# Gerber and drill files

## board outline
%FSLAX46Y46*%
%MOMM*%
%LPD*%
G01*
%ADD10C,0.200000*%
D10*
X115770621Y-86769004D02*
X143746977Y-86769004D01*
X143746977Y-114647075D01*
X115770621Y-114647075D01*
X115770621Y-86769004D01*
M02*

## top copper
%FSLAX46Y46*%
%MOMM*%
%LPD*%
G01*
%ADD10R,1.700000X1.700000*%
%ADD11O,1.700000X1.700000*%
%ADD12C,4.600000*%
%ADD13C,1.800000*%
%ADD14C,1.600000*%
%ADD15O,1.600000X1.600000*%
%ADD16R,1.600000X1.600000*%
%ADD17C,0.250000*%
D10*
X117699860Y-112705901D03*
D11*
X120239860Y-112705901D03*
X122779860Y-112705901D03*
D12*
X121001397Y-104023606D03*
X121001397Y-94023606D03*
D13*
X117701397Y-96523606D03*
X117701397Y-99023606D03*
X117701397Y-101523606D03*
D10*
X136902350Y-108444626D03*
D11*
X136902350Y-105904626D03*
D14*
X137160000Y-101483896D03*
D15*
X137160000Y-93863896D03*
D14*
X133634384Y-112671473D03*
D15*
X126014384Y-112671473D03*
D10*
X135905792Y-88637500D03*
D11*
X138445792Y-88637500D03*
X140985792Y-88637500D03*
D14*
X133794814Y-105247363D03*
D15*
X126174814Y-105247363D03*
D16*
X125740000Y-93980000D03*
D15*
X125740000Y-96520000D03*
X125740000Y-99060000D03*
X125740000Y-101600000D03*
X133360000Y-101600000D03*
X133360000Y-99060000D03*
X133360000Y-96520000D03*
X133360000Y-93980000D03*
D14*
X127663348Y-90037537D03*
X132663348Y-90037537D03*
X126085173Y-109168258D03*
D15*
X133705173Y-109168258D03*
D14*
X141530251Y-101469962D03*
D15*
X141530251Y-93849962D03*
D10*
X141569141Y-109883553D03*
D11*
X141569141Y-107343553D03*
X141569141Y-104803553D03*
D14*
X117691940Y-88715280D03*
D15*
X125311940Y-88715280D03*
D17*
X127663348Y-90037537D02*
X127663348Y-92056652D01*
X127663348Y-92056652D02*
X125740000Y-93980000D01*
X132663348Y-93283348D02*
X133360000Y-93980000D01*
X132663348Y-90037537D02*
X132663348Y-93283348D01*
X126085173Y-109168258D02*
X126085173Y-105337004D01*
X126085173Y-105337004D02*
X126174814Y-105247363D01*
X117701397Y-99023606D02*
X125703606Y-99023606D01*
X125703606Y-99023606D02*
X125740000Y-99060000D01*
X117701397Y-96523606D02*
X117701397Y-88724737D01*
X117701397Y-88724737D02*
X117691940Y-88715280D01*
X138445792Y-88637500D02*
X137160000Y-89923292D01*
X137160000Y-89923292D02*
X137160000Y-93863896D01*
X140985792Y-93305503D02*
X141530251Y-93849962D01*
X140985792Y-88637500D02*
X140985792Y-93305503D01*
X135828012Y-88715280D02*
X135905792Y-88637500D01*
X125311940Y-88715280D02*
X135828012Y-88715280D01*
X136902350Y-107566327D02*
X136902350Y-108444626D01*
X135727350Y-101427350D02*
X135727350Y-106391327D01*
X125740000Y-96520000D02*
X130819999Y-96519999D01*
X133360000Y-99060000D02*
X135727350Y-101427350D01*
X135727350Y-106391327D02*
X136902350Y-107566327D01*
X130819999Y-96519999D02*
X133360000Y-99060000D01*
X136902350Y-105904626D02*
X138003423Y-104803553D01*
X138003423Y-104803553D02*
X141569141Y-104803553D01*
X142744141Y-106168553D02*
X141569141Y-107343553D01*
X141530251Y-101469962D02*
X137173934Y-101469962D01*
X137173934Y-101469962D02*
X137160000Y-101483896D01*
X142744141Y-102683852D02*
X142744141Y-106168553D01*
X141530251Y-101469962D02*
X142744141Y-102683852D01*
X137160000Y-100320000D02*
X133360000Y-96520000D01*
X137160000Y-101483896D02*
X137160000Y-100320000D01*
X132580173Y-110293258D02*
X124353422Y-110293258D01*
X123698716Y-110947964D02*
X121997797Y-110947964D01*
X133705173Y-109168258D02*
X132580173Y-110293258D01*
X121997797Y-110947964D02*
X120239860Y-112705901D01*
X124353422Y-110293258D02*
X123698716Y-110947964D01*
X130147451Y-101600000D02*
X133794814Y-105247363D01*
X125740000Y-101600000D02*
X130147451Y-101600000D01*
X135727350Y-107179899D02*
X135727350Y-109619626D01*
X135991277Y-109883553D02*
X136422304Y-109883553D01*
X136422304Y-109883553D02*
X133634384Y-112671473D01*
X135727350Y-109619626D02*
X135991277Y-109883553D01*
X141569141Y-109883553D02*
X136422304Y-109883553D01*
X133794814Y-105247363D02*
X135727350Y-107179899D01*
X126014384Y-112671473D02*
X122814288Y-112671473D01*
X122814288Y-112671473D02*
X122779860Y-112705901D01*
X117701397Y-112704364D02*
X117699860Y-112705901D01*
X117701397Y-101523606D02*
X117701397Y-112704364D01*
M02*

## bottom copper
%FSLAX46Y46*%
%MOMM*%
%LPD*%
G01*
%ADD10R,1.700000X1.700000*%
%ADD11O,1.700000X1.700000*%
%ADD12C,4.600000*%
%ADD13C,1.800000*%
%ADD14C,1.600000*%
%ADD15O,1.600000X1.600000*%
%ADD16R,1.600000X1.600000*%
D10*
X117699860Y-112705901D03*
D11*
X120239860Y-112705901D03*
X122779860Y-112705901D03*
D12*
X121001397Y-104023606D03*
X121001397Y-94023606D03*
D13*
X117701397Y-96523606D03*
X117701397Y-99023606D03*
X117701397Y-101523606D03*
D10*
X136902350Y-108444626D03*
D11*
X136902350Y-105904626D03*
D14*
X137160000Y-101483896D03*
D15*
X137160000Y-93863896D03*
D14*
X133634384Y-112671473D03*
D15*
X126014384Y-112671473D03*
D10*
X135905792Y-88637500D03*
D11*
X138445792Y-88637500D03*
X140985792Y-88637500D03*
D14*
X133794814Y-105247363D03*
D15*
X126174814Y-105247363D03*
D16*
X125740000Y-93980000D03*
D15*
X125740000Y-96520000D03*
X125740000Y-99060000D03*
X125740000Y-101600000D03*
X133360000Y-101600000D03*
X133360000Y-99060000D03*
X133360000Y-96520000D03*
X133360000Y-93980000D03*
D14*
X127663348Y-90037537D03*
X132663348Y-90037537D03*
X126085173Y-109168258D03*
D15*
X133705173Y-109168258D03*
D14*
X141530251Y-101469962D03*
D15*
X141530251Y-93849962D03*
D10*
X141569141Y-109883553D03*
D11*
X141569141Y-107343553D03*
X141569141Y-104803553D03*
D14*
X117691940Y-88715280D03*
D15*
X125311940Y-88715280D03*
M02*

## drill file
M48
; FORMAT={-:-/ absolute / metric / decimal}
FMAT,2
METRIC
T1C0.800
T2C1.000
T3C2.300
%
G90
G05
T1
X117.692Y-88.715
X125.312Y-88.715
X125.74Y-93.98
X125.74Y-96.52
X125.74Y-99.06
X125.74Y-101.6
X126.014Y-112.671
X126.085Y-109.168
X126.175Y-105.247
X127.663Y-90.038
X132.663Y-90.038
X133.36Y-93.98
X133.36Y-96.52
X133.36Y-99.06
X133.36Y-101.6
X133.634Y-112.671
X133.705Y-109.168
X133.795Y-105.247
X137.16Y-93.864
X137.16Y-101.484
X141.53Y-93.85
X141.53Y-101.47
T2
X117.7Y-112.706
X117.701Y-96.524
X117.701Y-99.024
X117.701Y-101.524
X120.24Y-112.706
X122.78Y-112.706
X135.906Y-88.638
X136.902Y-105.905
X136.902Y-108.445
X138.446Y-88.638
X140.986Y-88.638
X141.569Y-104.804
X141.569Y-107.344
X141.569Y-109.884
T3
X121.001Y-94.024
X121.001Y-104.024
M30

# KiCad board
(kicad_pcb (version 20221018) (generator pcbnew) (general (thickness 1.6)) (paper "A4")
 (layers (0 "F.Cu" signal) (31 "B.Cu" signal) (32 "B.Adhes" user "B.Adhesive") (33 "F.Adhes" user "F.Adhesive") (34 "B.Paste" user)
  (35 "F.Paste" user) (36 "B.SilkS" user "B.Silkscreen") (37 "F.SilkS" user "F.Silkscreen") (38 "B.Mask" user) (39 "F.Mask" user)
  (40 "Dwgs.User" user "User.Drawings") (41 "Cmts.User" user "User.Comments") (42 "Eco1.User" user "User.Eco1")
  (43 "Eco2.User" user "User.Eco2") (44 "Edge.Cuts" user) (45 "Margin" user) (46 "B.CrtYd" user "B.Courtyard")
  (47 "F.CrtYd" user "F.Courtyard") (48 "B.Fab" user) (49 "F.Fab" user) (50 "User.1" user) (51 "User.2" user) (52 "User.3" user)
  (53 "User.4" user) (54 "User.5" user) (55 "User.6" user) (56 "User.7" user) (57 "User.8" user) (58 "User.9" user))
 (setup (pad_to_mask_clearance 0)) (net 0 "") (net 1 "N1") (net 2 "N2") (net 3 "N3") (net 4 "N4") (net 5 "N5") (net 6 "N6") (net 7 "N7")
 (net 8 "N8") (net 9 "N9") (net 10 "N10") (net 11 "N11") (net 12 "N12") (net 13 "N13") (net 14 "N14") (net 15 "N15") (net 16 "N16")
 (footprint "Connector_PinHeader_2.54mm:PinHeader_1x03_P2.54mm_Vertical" (layer "F.Cu") (at 117.69986 112.705901 90)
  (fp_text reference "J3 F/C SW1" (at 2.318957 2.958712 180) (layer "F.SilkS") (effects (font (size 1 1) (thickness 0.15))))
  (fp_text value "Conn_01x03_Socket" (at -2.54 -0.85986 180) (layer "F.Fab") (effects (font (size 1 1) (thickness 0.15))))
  (pad "1" thru_hole rect (at 0 0 90) (size 1.7 1.7) (drill 1) (layers "*.Cu" "*.Mask") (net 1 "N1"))
  (pad "2" thru_hole oval (at 0 2.54 90) (size 1.7 1.7) (drill 1) (layers "*.Cu" "*.Mask") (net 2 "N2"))
  (pad "3" thru_hole oval (at 0 5.08 90) (size 1.7 1.7) (drill 1) (layers "*.Cu" "*.Mask") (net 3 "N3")))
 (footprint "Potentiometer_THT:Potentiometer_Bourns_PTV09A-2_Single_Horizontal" (layer "F.Cu") (at 117.701397 96.523606 180)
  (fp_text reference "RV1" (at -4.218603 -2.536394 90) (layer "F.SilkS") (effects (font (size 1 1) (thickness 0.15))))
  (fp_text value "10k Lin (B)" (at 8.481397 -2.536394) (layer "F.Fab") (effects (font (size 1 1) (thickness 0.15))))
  (pad "" thru_hole circle (at -3.3 -7.5 180) (size 4.6 4.6) (drill 2.3) (layers "*.Cu" "*.Mask"))
  (pad "" thru_hole circle (at -3.3 2.5 180) (size 4.6 4.6) (drill 2.3) (layers "*.Cu" "*.Mask"))
  (pad "1" thru_hole circle (at 0 0 180) (size 1.8 1.8) (drill 1) (layers "*.Cu" "*.Mask") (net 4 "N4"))
  (pad "2" thru_hole circle (at 0 -2.5 180) (size 1.8 1.8) (drill 1) (layers "*.Cu" "*.Mask") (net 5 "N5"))
  (pad "3" thru_hole circle (at 0 -5 180) (size 1.8 1.8) (drill 1) (layers "*.Cu" "*.Mask") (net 1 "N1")))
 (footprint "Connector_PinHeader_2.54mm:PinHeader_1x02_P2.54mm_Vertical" (layer "F.Cu") (at 136.90235 108.444626 180)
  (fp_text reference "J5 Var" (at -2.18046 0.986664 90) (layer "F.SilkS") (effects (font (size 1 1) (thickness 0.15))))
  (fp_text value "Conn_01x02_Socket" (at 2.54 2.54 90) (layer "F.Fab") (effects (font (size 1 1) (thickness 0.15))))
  (pad "1" thru_hole rect (at 0 0 180) (size 1.7 1.7) (drill 1) (layers "*.Cu" "*.Mask") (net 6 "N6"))
  (pad "2" thru_hole oval (at 0 2.54 180) (size 1.7 1.7) (drill 1) (layers "*.Cu" "*.Mask") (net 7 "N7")))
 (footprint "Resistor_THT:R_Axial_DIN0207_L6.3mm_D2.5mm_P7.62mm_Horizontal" (layer "F.Cu") (at 137.16 101.483896 90)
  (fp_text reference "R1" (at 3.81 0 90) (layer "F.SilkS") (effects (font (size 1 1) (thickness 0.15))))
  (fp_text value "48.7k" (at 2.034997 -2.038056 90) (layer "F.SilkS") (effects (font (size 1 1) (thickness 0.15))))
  (pad "1" thru_hole circle (at 0 0 90) (size 1.6 1.6) (drill 0.8) (layers "*.Cu" "*.Mask") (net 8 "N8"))
  (pad "2" thru_hole oval (at 7.62 0 90) (size 1.6 1.6) (drill 0.8) (layers "*.Cu" "*.Mask") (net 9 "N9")))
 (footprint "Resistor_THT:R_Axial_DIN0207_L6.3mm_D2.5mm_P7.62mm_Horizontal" (layer "F.Cu") (at 133.634384 112.671473 180)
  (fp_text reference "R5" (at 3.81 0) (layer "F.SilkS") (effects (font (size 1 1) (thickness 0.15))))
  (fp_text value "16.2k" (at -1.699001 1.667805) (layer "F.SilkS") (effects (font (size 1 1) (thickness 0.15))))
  (pad "1" thru_hole circle (at 0 0 180) (size 1.6 1.6) (drill 0.8) (layers "*.Cu" "*.Mask") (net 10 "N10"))
  (pad "2" thru_hole oval (at 7.62 0 180) (size 1.6 1.6) (drill 0.8) (layers "*.Cu" "*.Mask") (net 3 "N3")))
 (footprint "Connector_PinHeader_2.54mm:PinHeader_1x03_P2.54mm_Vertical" (layer "F.Cu") (at 135.905792 88.6375 90)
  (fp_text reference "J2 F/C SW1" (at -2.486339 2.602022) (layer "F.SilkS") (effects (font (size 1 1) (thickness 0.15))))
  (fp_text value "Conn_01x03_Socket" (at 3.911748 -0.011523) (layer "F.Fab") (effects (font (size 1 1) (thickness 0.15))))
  (pad "1" thru_hole rect (at 0 0 90) (size 1.7 1.7) (drill 1) (layers "*.Cu" "*.Mask") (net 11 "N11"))
  (pad "2" thru_hole oval (at 0 2.54 90) (size 1.7 1.7) (drill 1) (layers "*.Cu" "*.Mask") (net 9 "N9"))
  (pad "3" thru_hole oval (at 0 5.08 90) (size 1.7 1.7) (drill 1) (layers "*.Cu" "*.Mask") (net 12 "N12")))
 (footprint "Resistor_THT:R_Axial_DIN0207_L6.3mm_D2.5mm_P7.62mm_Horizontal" (layer "F.Cu") (at 133.794814 105.247363 180)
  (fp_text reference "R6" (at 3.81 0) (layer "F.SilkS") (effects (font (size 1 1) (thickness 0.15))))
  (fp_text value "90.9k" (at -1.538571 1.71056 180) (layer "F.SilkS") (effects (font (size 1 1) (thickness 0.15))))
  (pad "1" thru_hole circle (at 0 0 180) (size 1.6 1.6) (drill 0.8) (layers "*.Cu" "*.Mask") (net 10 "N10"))
  (pad "2" thru_hole oval (at 7.62 0 180) (size 1.6 1.6) (drill 0.8) (layers "*.Cu" "*.Mask") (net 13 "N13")))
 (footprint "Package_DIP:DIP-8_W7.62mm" (layer "F.Cu") (at 125.74 93.98)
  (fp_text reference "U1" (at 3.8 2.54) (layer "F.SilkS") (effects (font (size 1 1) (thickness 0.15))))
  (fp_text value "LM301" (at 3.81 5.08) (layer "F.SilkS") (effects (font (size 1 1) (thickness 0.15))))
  (pad "1" thru_hole rect (at 0 0) (size 1.6 1.6) (drill 0.8) (layers "*.Cu" "*.Mask") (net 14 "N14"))
  (pad "2" thru_hole oval (at 0 2.54) (size 1.6 1.6) (drill 0.8) (layers "*.Cu" "*.Mask") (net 6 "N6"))
  (pad "3" thru_hole oval (at 0 5.08) (size 1.6 1.6) (drill 0.8) (layers "*.Cu" "*.Mask") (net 5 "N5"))
  (pad "4" thru_hole oval (at 0 7.62) (size 1.6 1.6) (drill 0.8) (layers "*.Cu" "*.Mask") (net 10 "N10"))
  (pad "5" thru_hole oval (at 7.62 7.62) (size 1.6 1.6) (drill 0.8) (layers "*.Cu" "*.Mask") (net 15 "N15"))
  (pad "6" thru_hole oval (at 7.62 5.08) (size 1.6 1.6) (drill 0.8) (layers "*.Cu" "*.Mask") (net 6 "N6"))
  (pad "7" thru_hole oval (at 7.62 2.54) (size 1.6 1.6) (drill 0.8) (layers "*.Cu" "*.Mask") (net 8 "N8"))
  (pad "8" thru_hole oval (at 7.62 0) (size 1.6 1.6) (drill 0.8) (layers "*.Cu" "*.Mask") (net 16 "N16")))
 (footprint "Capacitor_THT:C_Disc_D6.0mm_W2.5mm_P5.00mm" (layer "F.Cu") (at 127.663348 90.037537)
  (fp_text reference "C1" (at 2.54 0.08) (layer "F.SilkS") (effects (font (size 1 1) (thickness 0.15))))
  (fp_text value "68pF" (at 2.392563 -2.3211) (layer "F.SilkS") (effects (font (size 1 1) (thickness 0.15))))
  (pad "1" thru_hole circle (at 0 0) (size 1.6 1.6) (drill 0.8) (layers "*.Cu" "*.Mask") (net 14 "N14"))
  (pad "2" thru_hole circle (at 5 0) (size 1.6 1.6) (drill 0.8) (layers "*.Cu" "*.Mask") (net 16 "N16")))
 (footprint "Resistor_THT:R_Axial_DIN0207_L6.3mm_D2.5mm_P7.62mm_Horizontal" (layer "F.Cu") (at 126.085173 109.168258)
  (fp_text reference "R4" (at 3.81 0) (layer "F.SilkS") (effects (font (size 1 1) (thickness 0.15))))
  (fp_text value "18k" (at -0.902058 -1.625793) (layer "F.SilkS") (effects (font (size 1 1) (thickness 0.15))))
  (pad "1" thru_hole circle (at 0 0) (size 1.6 1.6) (drill 0.8) (layers "*.Cu" "*.Mask") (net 13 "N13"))
  (pad "2" thru_hole oval (at 7.62 0) (size 1.6 1.6) (drill 0.8) (layers "*.Cu" "*.Mask") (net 2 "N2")))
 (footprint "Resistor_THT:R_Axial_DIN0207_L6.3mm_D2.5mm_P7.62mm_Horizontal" (layer "F.Cu") (at 141.530251 101.469962 90)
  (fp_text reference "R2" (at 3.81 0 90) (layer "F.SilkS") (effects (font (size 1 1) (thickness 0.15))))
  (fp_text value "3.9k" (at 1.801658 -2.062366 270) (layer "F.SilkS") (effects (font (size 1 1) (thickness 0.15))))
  (pad "1" thru_hole circle (at 0 0 90) (size 1.6 1.6) (drill 0.8) (layers "*.Cu" "*.Mask") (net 8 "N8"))
  (pad "2" thru_hole oval (at 7.62 0 90) (size 1.6 1.6) (drill 0.8) (layers "*.Cu" "*.Mask") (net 12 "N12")))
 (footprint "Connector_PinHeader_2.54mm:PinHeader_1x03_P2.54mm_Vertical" (layer "F.Cu") (at 141.569141 109.883553 180)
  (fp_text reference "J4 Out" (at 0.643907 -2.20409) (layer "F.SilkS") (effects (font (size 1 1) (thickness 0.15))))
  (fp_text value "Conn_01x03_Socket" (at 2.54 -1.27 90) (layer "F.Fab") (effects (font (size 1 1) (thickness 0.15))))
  (pad "1" thru_hole rect (at 0 0 180) (size 1.7 1.7) (drill 1) (layers "*.Cu" "*.Mask") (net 10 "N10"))
  (pad "2" thru_hole oval (at 0 2.54 180) (size 1.7 1.7) (drill 1) (layers "*.Cu" "*.Mask") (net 8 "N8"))
  (pad "3" thru_hole oval (at 0 5.08 180) (size 1.7 1.7) (drill 1) (layers "*.Cu" "*.Mask") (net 7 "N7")))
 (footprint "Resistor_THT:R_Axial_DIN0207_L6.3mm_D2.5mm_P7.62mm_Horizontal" (layer "F.Cu") (at 117.69194 88.71528)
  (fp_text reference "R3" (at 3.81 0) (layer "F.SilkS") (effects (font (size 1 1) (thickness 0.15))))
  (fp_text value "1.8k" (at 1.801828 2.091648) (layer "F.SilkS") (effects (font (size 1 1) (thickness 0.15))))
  (pad "1" thru_hole circle (at 0 0) (size 1.6 1.6) (drill 0.8) (layers "*.Cu" "*.Mask") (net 4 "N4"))
  (pad "2" thru_hole oval (at 7.62 0) (size 1.6 1.6) (drill 0.8) (layers "*.Cu" "*.Mask") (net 11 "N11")))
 (gr_rect (start 115.770621 86.769004) (end 143.746977 114.647075) (stroke (width 0.2) (type solid)) (fill none) (layer "Edge.Cuts"))
 (segment (start 127.663348 90.037537) (end 127.663348 92.056652) (width 0.25) (layer "F.Cu") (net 14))
 (segment (start 127.663348 92.056652) (end 125.74 93.98) (width 0.25) (layer "F.Cu") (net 14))
 (segment (start 132.663348 93.283348) (end 133.36 93.98) (width 0.25) (layer "F.Cu") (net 16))
 (segment (start 132.663348 90.037537) (end 132.663348 93.283348) (width 0.25) (layer "F.Cu") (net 16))
 (segment (start 126.085173 109.168258) (end 126.085173 105.337004) (width 0.25) (layer "F.Cu") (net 13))
 (segment (start 126.085173 105.337004) (end 126.174814 105.247363) (width 0.25) (layer "F.Cu") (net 13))
 (segment (start 117.701397 99.023606) (end 125.703606 99.023606) (width 0.25) (layer "F.Cu") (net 5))
 (segment (start 125.703606 99.023606) (end 125.74 99.06) (width 0.25) (layer "F.Cu") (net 5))
 (segment (start 117.701397 96.523606) (end 117.701397 88.724737) (width 0.25) (layer "F.Cu") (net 4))
 (segment (start 117.701397 88.724737) (end 117.69194 88.71528) (width 0.25) (layer "F.Cu") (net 4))
 (segment (start 138.445792 88.6375) (end 137.16 89.923292) (width 0.25) (layer "F.Cu") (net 9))
 (segment (start 137.16 89.923292) (end 137.16 93.863896) (width 0.25) (layer "F.Cu") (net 9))
 (segment (start 140.985792 93.305503) (end 141.530251 93.849962) (width 0.25) (layer "F.Cu") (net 12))
 (segment (start 140.985792 88.6375) (end 140.985792 93.305503) (width 0.25) (layer "F.Cu") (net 12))
 (segment (start 135.828012 88.71528) (end 135.905792 88.6375) (width 0.25) (layer "F.Cu") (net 11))
 (segment (start 125.31194 88.71528) (end 135.828012 88.71528) (width 0.25) (layer "F.Cu") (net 11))
 (segment (start 136.90235 107.566327) (end 136.90235 108.444626) (width 0.25) (layer "F.Cu") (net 6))
 (segment (start 135.72735 101.42735) (end 135.72735 106.391327) (width 0.25) (layer "F.Cu") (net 6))
 (segment (start 125.74 96.52) (end 130.819999 96.519999) (width 0.25) (layer "F.Cu") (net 6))
 (segment (start 133.36 99.06) (end 135.72735 101.42735) (width 0.25) (layer "F.Cu") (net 6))
 (segment (start 135.72735 106.391327) (end 136.90235 107.566327) (width 0.25) (layer "F.Cu") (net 6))
 (segment (start 130.819999 96.519999) (end 133.36 99.06) (width 0.25) (layer "F.Cu") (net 6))
 (segment (start 136.90235 105.904626) (end 138.003423 104.803553) (width 0.25) (layer "F.Cu") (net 7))
 (segment (start 138.003423 104.803553) (end 141.569141 104.803553) (width 0.25) (layer "F.Cu") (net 7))
 (segment (start 142.744141 106.168553) (end 141.569141 107.343553) (width 0.25) (layer "F.Cu") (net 8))
 (segment (start 141.530251 101.469962) (end 137.173934 101.469962) (width 0.25) (layer "F.Cu") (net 8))
 (segment (start 137.173934 101.469962) (end 137.16 101.483896) (width 0.25) (layer "F.Cu") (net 8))
 (segment (start 142.744141 102.683852) (end 142.744141 106.168553) (width 0.25) (layer "F.Cu") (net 8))
 (segment (start 141.530251 101.469962) (end 142.744141 102.683852) (width 0.25) (layer "F.Cu") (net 8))
 (segment (start 137.16 100.32) (end 133.36 96.52) (width 0.25) (layer "F.Cu") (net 8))
 (segment (start 137.16 101.483896) (end 137.16 100.32) (width 0.25) (layer "F.Cu") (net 8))
 (segment (start 132.580173 110.293258) (end 124.353422 110.293258) (width 0.25) (layer "F.Cu") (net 2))
 (segment (start 123.698716 110.947964) (end 121.997797 110.947964) (width 0.25) (layer "F.Cu") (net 2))
 (segment (start 133.705173 109.168258) (end 132.580173 110.293258) (width 0.25) (layer "F.Cu") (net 2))
 (segment (start 121.997797 110.947964) (end 120.23986 112.705901) (width 0.25) (layer "F.Cu") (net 2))
 (segment (start 124.353422 110.293258) (end 123.698716 110.947964) (width 0.25) (layer "F.Cu") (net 2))
 (segment (start 130.147451 101.6) (end 133.794814 105.247363) (width 0.25) (layer "F.Cu") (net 10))
 (segment (start 125.74 101.6) (end 130.147451 101.6) (width 0.25) (layer "F.Cu") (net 10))
 (segment (start 135.72735 107.179899) (end 135.72735 109.619626) (width 0.25) (layer "F.Cu") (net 10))
 (segment (start 135.991277 109.883553) (end 136.422304 109.883553) (width 0.25) (layer "F.Cu") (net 10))
 (segment (start 136.422304 109.883553) (end 133.634384 112.671473) (width 0.25) (layer "F.Cu") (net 10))
 (segment (start 135.72735 109.619626) (end 135.991277 109.883553) (width 0.25) (layer "F.Cu") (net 10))
 (segment (start 141.569141 109.883553) (end 136.422304 109.883553) (width 0.25) (layer "F.Cu") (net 10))
 (segment (start 133.794814 105.247363) (end 135.72735 107.179899) (width 0.25) (layer "F.Cu") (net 10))
 (segment (start 126.014384 112.671473) (end 122.814288 112.671473) (width 0.25) (layer "F.Cu") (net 3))
 (segment (start 122.814288 112.671473) (end 122.77986 112.705901) (width 0.25) (layer "F.Cu") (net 3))
 (segment (start 117.701397 112.704364) (end 117.69986 112.705901) (width 0.25) (layer "F.Cu") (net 1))
 (segment (start 117.701397 101.523606) (end 117.701397 112.704364) (width 0.25) (layer "F.Cu") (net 1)))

